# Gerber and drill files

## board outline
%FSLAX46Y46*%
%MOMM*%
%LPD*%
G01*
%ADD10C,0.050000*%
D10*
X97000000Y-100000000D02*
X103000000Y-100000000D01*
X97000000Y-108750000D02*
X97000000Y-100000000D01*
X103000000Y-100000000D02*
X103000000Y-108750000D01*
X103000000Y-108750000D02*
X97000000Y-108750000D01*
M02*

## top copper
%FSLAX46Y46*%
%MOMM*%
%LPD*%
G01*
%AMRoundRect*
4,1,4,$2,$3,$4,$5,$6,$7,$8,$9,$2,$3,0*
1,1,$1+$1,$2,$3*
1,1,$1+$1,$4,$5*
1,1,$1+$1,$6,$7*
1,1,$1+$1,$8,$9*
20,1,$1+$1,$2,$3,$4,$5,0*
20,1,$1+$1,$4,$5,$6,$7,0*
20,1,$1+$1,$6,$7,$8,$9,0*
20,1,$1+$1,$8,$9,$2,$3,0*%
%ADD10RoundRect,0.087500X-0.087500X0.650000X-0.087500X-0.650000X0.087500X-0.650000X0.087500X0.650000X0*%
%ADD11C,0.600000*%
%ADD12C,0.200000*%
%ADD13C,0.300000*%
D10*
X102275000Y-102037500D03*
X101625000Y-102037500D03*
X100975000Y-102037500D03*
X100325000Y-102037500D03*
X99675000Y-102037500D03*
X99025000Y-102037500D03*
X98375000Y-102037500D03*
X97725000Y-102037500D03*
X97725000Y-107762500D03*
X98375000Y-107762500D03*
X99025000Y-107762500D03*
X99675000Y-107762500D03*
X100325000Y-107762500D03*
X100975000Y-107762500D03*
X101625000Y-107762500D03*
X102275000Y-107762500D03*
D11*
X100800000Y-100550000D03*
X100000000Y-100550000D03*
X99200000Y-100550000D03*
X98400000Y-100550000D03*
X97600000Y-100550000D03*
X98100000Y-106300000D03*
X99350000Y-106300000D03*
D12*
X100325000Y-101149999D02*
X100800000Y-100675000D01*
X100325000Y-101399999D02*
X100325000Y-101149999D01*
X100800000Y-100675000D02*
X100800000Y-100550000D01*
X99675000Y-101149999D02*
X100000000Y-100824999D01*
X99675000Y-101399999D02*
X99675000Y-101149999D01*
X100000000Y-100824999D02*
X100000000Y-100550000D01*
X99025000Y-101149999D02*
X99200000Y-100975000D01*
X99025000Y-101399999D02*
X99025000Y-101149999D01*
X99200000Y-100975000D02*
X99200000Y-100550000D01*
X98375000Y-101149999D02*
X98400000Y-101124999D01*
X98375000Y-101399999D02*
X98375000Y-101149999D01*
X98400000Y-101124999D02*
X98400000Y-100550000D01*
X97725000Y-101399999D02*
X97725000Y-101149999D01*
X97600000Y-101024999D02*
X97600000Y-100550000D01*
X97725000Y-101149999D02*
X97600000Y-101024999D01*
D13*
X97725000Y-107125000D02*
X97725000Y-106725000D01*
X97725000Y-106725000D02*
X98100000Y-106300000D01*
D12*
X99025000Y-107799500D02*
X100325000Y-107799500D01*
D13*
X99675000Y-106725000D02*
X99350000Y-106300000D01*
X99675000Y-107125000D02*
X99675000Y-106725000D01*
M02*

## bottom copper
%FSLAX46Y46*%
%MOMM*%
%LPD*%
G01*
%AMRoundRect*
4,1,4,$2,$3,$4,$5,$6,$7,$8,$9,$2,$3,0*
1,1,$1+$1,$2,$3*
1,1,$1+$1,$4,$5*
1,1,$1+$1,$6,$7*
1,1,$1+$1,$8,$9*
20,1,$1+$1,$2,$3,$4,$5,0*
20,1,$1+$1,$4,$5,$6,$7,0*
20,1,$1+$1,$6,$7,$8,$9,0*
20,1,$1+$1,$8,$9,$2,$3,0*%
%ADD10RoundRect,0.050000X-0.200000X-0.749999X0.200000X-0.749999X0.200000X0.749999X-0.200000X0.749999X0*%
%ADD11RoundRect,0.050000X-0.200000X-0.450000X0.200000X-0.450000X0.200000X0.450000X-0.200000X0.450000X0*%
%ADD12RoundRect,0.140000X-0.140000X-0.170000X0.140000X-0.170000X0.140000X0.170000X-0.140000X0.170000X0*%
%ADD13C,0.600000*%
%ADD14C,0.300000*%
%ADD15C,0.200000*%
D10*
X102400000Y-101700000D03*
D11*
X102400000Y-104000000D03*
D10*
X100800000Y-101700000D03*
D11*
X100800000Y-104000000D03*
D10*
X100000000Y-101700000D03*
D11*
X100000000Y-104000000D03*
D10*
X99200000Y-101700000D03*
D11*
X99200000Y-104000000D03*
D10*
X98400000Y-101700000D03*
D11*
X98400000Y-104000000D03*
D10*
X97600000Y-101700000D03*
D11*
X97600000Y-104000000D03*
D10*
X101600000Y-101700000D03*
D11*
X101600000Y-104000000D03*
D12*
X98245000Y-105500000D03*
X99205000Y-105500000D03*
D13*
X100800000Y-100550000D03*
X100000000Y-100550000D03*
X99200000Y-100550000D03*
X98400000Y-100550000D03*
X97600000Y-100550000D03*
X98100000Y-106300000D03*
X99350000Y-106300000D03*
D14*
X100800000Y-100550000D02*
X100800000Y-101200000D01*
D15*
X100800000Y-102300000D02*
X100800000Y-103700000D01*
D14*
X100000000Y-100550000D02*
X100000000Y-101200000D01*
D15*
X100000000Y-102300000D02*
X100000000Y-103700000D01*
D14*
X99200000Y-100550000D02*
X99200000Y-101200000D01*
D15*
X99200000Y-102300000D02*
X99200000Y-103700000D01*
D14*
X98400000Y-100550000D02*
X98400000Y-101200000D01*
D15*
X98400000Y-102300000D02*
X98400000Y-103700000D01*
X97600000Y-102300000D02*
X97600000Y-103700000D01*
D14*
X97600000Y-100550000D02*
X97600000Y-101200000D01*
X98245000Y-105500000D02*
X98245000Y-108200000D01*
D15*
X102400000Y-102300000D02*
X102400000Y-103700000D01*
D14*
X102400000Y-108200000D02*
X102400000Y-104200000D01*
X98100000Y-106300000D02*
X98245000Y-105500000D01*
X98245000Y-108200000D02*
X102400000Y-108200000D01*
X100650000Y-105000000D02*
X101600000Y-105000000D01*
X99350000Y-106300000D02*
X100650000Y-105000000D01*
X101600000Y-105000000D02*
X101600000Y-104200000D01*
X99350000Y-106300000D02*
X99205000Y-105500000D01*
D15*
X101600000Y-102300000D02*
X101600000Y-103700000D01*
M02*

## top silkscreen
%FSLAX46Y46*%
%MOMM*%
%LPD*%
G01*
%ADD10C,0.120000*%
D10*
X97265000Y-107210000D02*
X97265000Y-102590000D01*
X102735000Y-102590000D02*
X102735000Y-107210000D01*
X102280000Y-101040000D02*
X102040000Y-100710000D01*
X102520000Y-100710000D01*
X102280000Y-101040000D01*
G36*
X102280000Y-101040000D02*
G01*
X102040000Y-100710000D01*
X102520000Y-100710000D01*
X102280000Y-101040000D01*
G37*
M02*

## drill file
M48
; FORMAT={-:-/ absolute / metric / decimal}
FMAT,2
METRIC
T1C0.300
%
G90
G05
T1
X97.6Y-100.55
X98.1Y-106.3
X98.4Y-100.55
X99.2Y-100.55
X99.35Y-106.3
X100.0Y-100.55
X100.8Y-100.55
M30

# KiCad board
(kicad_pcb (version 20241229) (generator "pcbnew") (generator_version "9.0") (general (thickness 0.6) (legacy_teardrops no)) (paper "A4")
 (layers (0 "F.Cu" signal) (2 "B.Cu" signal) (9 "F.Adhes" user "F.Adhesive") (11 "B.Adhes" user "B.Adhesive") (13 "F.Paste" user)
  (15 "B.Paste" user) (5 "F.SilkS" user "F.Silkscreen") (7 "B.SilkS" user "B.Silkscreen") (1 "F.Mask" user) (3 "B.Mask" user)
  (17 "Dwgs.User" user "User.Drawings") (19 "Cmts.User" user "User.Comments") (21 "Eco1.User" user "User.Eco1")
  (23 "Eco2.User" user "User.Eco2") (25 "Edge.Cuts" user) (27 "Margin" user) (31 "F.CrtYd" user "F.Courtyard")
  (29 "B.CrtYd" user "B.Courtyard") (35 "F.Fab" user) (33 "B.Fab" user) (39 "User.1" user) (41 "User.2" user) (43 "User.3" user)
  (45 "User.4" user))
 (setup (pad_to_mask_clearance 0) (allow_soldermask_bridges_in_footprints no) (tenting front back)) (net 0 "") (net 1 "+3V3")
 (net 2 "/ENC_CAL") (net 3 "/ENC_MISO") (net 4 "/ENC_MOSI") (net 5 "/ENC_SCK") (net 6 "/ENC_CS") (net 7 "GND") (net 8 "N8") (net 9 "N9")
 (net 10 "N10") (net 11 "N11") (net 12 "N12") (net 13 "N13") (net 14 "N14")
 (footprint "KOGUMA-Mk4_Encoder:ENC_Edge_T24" (layer "F.Cu") (at 100 100)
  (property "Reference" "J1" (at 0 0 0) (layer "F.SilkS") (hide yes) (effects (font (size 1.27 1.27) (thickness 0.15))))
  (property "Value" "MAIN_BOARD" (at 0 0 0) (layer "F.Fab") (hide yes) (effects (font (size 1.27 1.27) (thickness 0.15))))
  (pad "1" smd roundrect (at 2.4 1.7) (size 0.5 1.599999) (layers "B.Cu" "B.Mask" "B.Paste") (roundrect_rratio 0.1) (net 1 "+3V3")
   (thermal_bridge_angle 45))
  (pad "1" smd roundrect (at 2.4 4) (size 0.5 1) (layers "B.Cu" "B.Mask" "B.Paste") (roundrect_rratio 0.1) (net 1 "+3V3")
   (thermal_bridge_angle 45))
  (pad "2" smd roundrect (at 0.8 1.7) (size 0.5 1.599999) (layers "B.Cu" "B.Mask" "B.Paste") (roundrect_rratio 0.1) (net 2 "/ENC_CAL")
   (thermal_bridge_angle 45))
  (pad "2" smd roundrect (at 0.8 4) (size 0.5 1) (layers "B.Cu" "B.Mask" "B.Paste") (roundrect_rratio 0.1) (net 2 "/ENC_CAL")
   (thermal_bridge_angle 45))
  (pad "3" smd roundrect (at 0 1.7) (size 0.5 1.599999) (layers "B.Cu" "B.Mask" "B.Paste") (roundrect_rratio 0.1) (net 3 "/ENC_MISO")
   (thermal_bridge_angle 45))
  (pad "3" smd roundrect (at 0 4) (size 0.5 1) (layers "B.Cu" "B.Mask" "B.Paste") (roundrect_rratio 0.1) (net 3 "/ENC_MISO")
   (thermal_bridge_angle 45))
  (pad "4" smd roundrect (at -0.8 1.7) (size 0.5 1.599999) (layers "B.Cu" "B.Mask" "B.Paste") (roundrect_rratio 0.1) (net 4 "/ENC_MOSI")
   (thermal_bridge_angle 45))
  (pad "4" smd roundrect (at -0.8 4) (size 0.5 1) (layers "B.Cu" "B.Mask" "B.Paste") (roundrect_rratio 0.1) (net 4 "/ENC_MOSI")
   (thermal_bridge_angle 45))
  (pad "5" smd roundrect (at -1.6 1.7) (size 0.5 1.599999) (layers "B.Cu" "B.Mask" "B.Paste") (roundrect_rratio 0.1) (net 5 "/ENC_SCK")
   (thermal_bridge_angle 45))
  (pad "5" smd roundrect (at -1.6 4) (size 0.5 1) (layers "B.Cu" "B.Mask" "B.Paste") (roundrect_rratio 0.1) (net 5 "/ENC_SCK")
   (thermal_bridge_angle 45))
  (pad "6" smd roundrect (at -2.4 1.7) (size 0.5 1.599999) (layers "B.Cu" "B.Mask" "B.Paste") (roundrect_rratio 0.1) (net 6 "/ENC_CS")
   (thermal_bridge_angle 45))
  (pad "6" smd roundrect (at -2.4 4) (size 0.5 1) (layers "B.Cu" "B.Mask" "B.Paste") (roundrect_rratio 0.1) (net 6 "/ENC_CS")
   (thermal_bridge_angle 45))
  (pad "7" smd roundrect (at 1.6 1.7) (size 0.5 1.599999) (layers "B.Cu" "B.Mask" "B.Paste") (roundrect_rratio 0.1) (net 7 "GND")
   (thermal_bridge_angle 45))
  (pad "7" smd roundrect (at 1.6 4) (size 0.5 1) (layers "B.Cu" "B.Mask" "B.Paste") (roundrect_rratio 0.1) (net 7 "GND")
   (thermal_bridge_angle 45)))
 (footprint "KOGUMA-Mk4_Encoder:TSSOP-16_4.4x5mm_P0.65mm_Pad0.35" (layer "F.Cu") (at 100 104.9 -90)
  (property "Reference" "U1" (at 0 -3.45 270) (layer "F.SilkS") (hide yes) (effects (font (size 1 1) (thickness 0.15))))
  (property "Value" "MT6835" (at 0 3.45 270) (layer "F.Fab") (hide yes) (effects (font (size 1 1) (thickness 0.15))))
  (fp_line (start 2.31 2.735) (end -2.31 2.735) (stroke (width 0.12) (type solid)) (layer "F.SilkS"))
  (fp_line (start -2.31 -2.735) (end 2.31 -2.735) (stroke (width 0.12) (type solid)) (layer "F.SilkS"))
  (fp_poly (pts (xy -3.86 -2.28) (xy -4.19 -2.04) (xy -4.19 -2.52)) (stroke (width 0.12) (type solid)) (fill yes) (layer "F.SilkS"))
  (pad "1" smd roundrect (at -2.8625 -2.275 270) (size 1.475 0.35) (layers "F.Cu" "F.Mask" "F.Paste") (roundrect_rratio 0.25) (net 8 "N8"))
  (pad "2" smd roundrect (at -2.8625 -1.625 270) (size 1.475 0.35) (layers "F.Cu" "F.Mask" "F.Paste") (roundrect_rratio 0.25) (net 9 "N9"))
  (pad "3" smd roundrect (at -2.8625 -0.975 270) (size 1.475 0.35) (layers "F.Cu" "F.Mask" "F.Paste") (roundrect_rratio 0.25) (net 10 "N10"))
  (pad "4" smd roundrect (at -2.8625 -0.325 270) (size 1.475 0.35) (layers "F.Cu" "F.Mask" "F.Paste") (roundrect_rratio 0.25)
   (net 2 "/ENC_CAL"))
  (pad "5" smd roundrect (at -2.8625 0.325 270) (size 1.475 0.35) (layers "F.Cu" "F.Mask" "F.Paste") (roundrect_rratio 0.25)
   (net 3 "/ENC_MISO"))
  (pad "6" smd roundrect (at -2.8625 0.975 270) (size 1.475 0.35) (layers "F.Cu" "F.Mask" "F.Paste") (roundrect_rratio 0.25)
   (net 4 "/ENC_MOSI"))
  (pad "7" smd roundrect (at -2.8625 1.625 270) (size 1.475 0.35) (layers "F.Cu" "F.Mask" "F.Paste") (roundrect_rratio 0.25)
   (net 5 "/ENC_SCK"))
  (pad "8" smd roundrect (at -2.8625 2.275 270) (size 1.475 0.35) (layers "F.Cu" "F.Mask" "F.Paste") (roundrect_rratio 0.25)
   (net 6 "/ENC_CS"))
  (pad "9" smd roundrect (at 2.8625 2.275 270) (size 1.475 0.35) (layers "F.Cu" "F.Mask" "F.Paste") (roundrect_rratio 0.25) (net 1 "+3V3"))
  (pad "10" smd roundrect (at 2.8625 1.625 270) (size 1.475 0.35) (layers "F.Cu" "F.Mask" "F.Paste") (roundrect_rratio 0.25) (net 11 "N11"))
  (pad "11" smd roundrect (at 2.8625 0.975 270) (size 1.475 0.35) (layers "F.Cu" "F.Mask" "F.Paste") (roundrect_rratio 0.25) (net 7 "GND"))
  (pad "12" smd roundrect (at 2.8625 0.325 270) (size 1.475 0.35) (layers "F.Cu" "F.Mask" "F.Paste") (roundrect_rratio 0.25) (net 7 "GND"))
  (pad "13" smd roundrect (at 2.8625 -0.325 270) (size 1.475 0.35) (layers "F.Cu" "F.Mask" "F.Paste") (roundrect_rratio 0.25) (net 7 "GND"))
  (pad "14" smd roundrect (at 2.8625 -0.975 270) (size 1.475 0.35) (layers "F.Cu" "F.Mask" "F.Paste") (roundrect_rratio 0.25) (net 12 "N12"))
  (pad "15" smd roundrect (at 2.8625 -1.625 270) (size 1.475 0.35) (layers "F.Cu" "F.Mask" "F.Paste") (roundrect_rratio 0.25) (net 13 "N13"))
  (pad "16" smd roundrect (at 2.8625 -2.275 270) (size 1.475 0.35) (layers "F.Cu" "F.Mask" "F.Paste") (roundrect_rratio 0.25) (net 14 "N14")))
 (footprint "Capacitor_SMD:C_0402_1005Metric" (layer "B.Cu") (at 98.725 105.5)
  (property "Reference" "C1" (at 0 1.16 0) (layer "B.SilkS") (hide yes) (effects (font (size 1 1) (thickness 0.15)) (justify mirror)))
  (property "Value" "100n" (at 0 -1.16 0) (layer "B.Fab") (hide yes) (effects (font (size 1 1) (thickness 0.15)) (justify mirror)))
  (pad "1" smd roundrect (at -0.48 0) (size 0.56 0.62) (layers "B.Cu" "B.Mask" "B.Paste") (roundrect_rratio 0.25) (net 1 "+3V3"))
  (pad "2" smd roundrect (at 0.48 0) (size 0.56 0.62) (layers "B.Cu" "B.Mask" "B.Paste") (roundrect_rratio 0.25) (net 7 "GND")))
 (gr_line (start 97 100) (end 103 100) (stroke (width 0.05) (type default)) (layer "Edge.Cuts"))
 (gr_line (start 97 108.75) (end 97 100) (stroke (width 0.05) (type default)) (layer "Edge.Cuts"))
 (gr_line (start 103 100) (end 103 108.75) (stroke (width 0.05) (type default)) (layer "Edge.Cuts"))
 (gr_line (start 103 108.75) (end 97 108.75) (stroke (width 0.05) (type default)) (layer "Edge.Cuts"))
 (segment (start 100.325 101.149999) (end 100.8 100.675) (width 0.2) (layer "F.Cu") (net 2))
 (segment (start 100.325 101.399999) (end 100.325 101.149999) (width 0.2) (layer "F.Cu") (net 2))
 (segment (start 100.8 100.675) (end 100.8 100.55) (width 0.2) (layer "F.Cu") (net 2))
 (via (at 100.8 100.55) (size 0.6) (drill 0.3) (layers "F.Cu" "B.Cu") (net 2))
 (segment (start 100.8 100.55) (end 100.8 101.2) (width 0.3) (layer "B.Cu") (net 2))
 (segment (start 100.8 102.3) (end 100.8 103.7) (width 0.2) (layer "B.Cu") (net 2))
 (segment (start 99.675 101.149999) (end 100 100.824999) (width 0.2) (layer "F.Cu") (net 3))
 (segment (start 99.675 101.399999) (end 99.675 101.149999) (width 0.2) (layer "F.Cu") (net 3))
 (segment (start 100 100.824999) (end 100 100.55) (width 0.2) (layer "F.Cu") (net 3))
 (via (at 100 100.55) (size 0.6) (drill 0.3) (layers "F.Cu" "B.Cu") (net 3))
 (segment (start 100 100.55) (end 100 101.2) (width 0.3) (layer "B.Cu") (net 3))
 (segment (start 100 102.3) (end 100 103.7) (width 0.2) (layer "B.Cu") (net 3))
 (segment (start 99.025 101.149999) (end 99.2 100.975) (width 0.2) (layer "F.Cu") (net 4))
 (segment (start 99.025 101.399999) (end 99.025 101.149999) (width 0.2) (layer "F.Cu") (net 4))
 (segment (start 99.2 100.975) (end 99.2 100.55) (width 0.2) (layer "F.Cu") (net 4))
 (via (at 99.2 100.55) (size 0.6) (drill 0.3) (layers "F.Cu" "B.Cu") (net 4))
 (segment (start 99.2 100.55) (end 99.2 101.2) (width 0.3) (layer "B.Cu") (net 4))
 (segment (start 99.2 102.3) (end 99.2 103.7) (width 0.2) (layer "B.Cu") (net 4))
 (segment (start 98.375 101.149999) (end 98.4 101.124999) (width 0.2) (layer "F.Cu") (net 5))
 (segment (start 98.375 101.399999) (end 98.375 101.149999) (width 0.2) (layer "F.Cu") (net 5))
 (segment (start 98.4 101.124999) (end 98.4 100.55) (width 0.2) (layer "F.Cu") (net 5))
 (via (at 98.4 100.55) (size 0.6) (drill 0.3) (layers "F.Cu" "B.Cu") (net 5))
 (segment (start 98.4 100.55) (end 98.4 101.2) (width 0.3) (layer "B.Cu") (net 5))
 (segment (start 98.4 102.3) (end 98.4 103.7) (width 0.2) (layer "B.Cu") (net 5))
 (segment (start 97.725 101.399999) (end 97.725 101.149999) (width 0.2) (layer "F.Cu") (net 6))
 (segment (start 97.6 101.024999) (end 97.6 100.55) (width 0.2) (layer "F.Cu") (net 6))
 (segment (start 97.725 101.149999) (end 97.6 101.024999) (width 0.2) (layer "F.Cu") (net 6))
 (via (at 97.6 100.55) (size 0.6) (drill 0.3) (layers "F.Cu" "B.Cu") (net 6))
 (segment (start 97.6 102.3) (end 97.6 103.7) (width 0.2) (layer "B.Cu") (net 6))
 (segment (start 97.6 100.55) (end 97.6 101.2) (width 0.3) (layer "B.Cu") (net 6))
 (segment (start 97.725 107.125) (end 97.725 106.725) (width 0.3) (layer "F.Cu") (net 1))
 (segment (start 97.725 106.725) (end 98.1 106.3) (width 0.3) (layer "F.Cu") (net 1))
 (via (at 98.1 106.3) (size 0.6) (drill 0.3) (layers "F.Cu" "B.Cu") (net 1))
 (segment (start 98.245 105.5) (end 98.245 108.2) (width 0.3) (layer "B.Cu") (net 1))
 (segment (start 102.4 102.3) (end 102.4 103.7) (width 0.2) (layer "B.Cu") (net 1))
 (segment (start 102.4 108.2) (end 102.4 104.2) (width 0.3) (layer "B.Cu") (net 1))
 (segment (start 98.1 106.3) (end 98.245 105.5) (width 0.3) (layer "B.Cu") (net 1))
 (segment (start 98.245 108.2) (end 102.4 108.2) (width 0.3) (layer "B.Cu") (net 1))
 (segment (start 99.025 107.7995) (end 100.325 107.7995) (width 0.2) (layer "F.Cu") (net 7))
 (segment (start 99.675 106.725) (end 99.35 106.3) (width 0.3) (layer "F.Cu") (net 7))
 (segment (start 99.675 107.125) (end 99.675 106.725) (width 0.3) (layer "F.Cu") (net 7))
 (via (at 99.35 106.3) (size 0.6) (drill 0.3) (layers "F.Cu" "B.Cu") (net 7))
 (segment (start 100.65 105) (end 101.6 105) (width 0.3) (layer "B.Cu") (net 7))
 (segment (start 99.35 106.3) (end 100.65 105) (width 0.3) (layer "B.Cu") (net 7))
 (segment (start 101.6 105) (end 101.6 104.2) (width 0.3) (layer "B.Cu") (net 7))
 (segment (start 99.35 106.3) (end 99.205 105.5) (width 0.3) (layer "B.Cu") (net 7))
 (segment (start 101.6 102.3) (end 101.6 103.7) (width 0.2) (layer "B.Cu") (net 7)))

